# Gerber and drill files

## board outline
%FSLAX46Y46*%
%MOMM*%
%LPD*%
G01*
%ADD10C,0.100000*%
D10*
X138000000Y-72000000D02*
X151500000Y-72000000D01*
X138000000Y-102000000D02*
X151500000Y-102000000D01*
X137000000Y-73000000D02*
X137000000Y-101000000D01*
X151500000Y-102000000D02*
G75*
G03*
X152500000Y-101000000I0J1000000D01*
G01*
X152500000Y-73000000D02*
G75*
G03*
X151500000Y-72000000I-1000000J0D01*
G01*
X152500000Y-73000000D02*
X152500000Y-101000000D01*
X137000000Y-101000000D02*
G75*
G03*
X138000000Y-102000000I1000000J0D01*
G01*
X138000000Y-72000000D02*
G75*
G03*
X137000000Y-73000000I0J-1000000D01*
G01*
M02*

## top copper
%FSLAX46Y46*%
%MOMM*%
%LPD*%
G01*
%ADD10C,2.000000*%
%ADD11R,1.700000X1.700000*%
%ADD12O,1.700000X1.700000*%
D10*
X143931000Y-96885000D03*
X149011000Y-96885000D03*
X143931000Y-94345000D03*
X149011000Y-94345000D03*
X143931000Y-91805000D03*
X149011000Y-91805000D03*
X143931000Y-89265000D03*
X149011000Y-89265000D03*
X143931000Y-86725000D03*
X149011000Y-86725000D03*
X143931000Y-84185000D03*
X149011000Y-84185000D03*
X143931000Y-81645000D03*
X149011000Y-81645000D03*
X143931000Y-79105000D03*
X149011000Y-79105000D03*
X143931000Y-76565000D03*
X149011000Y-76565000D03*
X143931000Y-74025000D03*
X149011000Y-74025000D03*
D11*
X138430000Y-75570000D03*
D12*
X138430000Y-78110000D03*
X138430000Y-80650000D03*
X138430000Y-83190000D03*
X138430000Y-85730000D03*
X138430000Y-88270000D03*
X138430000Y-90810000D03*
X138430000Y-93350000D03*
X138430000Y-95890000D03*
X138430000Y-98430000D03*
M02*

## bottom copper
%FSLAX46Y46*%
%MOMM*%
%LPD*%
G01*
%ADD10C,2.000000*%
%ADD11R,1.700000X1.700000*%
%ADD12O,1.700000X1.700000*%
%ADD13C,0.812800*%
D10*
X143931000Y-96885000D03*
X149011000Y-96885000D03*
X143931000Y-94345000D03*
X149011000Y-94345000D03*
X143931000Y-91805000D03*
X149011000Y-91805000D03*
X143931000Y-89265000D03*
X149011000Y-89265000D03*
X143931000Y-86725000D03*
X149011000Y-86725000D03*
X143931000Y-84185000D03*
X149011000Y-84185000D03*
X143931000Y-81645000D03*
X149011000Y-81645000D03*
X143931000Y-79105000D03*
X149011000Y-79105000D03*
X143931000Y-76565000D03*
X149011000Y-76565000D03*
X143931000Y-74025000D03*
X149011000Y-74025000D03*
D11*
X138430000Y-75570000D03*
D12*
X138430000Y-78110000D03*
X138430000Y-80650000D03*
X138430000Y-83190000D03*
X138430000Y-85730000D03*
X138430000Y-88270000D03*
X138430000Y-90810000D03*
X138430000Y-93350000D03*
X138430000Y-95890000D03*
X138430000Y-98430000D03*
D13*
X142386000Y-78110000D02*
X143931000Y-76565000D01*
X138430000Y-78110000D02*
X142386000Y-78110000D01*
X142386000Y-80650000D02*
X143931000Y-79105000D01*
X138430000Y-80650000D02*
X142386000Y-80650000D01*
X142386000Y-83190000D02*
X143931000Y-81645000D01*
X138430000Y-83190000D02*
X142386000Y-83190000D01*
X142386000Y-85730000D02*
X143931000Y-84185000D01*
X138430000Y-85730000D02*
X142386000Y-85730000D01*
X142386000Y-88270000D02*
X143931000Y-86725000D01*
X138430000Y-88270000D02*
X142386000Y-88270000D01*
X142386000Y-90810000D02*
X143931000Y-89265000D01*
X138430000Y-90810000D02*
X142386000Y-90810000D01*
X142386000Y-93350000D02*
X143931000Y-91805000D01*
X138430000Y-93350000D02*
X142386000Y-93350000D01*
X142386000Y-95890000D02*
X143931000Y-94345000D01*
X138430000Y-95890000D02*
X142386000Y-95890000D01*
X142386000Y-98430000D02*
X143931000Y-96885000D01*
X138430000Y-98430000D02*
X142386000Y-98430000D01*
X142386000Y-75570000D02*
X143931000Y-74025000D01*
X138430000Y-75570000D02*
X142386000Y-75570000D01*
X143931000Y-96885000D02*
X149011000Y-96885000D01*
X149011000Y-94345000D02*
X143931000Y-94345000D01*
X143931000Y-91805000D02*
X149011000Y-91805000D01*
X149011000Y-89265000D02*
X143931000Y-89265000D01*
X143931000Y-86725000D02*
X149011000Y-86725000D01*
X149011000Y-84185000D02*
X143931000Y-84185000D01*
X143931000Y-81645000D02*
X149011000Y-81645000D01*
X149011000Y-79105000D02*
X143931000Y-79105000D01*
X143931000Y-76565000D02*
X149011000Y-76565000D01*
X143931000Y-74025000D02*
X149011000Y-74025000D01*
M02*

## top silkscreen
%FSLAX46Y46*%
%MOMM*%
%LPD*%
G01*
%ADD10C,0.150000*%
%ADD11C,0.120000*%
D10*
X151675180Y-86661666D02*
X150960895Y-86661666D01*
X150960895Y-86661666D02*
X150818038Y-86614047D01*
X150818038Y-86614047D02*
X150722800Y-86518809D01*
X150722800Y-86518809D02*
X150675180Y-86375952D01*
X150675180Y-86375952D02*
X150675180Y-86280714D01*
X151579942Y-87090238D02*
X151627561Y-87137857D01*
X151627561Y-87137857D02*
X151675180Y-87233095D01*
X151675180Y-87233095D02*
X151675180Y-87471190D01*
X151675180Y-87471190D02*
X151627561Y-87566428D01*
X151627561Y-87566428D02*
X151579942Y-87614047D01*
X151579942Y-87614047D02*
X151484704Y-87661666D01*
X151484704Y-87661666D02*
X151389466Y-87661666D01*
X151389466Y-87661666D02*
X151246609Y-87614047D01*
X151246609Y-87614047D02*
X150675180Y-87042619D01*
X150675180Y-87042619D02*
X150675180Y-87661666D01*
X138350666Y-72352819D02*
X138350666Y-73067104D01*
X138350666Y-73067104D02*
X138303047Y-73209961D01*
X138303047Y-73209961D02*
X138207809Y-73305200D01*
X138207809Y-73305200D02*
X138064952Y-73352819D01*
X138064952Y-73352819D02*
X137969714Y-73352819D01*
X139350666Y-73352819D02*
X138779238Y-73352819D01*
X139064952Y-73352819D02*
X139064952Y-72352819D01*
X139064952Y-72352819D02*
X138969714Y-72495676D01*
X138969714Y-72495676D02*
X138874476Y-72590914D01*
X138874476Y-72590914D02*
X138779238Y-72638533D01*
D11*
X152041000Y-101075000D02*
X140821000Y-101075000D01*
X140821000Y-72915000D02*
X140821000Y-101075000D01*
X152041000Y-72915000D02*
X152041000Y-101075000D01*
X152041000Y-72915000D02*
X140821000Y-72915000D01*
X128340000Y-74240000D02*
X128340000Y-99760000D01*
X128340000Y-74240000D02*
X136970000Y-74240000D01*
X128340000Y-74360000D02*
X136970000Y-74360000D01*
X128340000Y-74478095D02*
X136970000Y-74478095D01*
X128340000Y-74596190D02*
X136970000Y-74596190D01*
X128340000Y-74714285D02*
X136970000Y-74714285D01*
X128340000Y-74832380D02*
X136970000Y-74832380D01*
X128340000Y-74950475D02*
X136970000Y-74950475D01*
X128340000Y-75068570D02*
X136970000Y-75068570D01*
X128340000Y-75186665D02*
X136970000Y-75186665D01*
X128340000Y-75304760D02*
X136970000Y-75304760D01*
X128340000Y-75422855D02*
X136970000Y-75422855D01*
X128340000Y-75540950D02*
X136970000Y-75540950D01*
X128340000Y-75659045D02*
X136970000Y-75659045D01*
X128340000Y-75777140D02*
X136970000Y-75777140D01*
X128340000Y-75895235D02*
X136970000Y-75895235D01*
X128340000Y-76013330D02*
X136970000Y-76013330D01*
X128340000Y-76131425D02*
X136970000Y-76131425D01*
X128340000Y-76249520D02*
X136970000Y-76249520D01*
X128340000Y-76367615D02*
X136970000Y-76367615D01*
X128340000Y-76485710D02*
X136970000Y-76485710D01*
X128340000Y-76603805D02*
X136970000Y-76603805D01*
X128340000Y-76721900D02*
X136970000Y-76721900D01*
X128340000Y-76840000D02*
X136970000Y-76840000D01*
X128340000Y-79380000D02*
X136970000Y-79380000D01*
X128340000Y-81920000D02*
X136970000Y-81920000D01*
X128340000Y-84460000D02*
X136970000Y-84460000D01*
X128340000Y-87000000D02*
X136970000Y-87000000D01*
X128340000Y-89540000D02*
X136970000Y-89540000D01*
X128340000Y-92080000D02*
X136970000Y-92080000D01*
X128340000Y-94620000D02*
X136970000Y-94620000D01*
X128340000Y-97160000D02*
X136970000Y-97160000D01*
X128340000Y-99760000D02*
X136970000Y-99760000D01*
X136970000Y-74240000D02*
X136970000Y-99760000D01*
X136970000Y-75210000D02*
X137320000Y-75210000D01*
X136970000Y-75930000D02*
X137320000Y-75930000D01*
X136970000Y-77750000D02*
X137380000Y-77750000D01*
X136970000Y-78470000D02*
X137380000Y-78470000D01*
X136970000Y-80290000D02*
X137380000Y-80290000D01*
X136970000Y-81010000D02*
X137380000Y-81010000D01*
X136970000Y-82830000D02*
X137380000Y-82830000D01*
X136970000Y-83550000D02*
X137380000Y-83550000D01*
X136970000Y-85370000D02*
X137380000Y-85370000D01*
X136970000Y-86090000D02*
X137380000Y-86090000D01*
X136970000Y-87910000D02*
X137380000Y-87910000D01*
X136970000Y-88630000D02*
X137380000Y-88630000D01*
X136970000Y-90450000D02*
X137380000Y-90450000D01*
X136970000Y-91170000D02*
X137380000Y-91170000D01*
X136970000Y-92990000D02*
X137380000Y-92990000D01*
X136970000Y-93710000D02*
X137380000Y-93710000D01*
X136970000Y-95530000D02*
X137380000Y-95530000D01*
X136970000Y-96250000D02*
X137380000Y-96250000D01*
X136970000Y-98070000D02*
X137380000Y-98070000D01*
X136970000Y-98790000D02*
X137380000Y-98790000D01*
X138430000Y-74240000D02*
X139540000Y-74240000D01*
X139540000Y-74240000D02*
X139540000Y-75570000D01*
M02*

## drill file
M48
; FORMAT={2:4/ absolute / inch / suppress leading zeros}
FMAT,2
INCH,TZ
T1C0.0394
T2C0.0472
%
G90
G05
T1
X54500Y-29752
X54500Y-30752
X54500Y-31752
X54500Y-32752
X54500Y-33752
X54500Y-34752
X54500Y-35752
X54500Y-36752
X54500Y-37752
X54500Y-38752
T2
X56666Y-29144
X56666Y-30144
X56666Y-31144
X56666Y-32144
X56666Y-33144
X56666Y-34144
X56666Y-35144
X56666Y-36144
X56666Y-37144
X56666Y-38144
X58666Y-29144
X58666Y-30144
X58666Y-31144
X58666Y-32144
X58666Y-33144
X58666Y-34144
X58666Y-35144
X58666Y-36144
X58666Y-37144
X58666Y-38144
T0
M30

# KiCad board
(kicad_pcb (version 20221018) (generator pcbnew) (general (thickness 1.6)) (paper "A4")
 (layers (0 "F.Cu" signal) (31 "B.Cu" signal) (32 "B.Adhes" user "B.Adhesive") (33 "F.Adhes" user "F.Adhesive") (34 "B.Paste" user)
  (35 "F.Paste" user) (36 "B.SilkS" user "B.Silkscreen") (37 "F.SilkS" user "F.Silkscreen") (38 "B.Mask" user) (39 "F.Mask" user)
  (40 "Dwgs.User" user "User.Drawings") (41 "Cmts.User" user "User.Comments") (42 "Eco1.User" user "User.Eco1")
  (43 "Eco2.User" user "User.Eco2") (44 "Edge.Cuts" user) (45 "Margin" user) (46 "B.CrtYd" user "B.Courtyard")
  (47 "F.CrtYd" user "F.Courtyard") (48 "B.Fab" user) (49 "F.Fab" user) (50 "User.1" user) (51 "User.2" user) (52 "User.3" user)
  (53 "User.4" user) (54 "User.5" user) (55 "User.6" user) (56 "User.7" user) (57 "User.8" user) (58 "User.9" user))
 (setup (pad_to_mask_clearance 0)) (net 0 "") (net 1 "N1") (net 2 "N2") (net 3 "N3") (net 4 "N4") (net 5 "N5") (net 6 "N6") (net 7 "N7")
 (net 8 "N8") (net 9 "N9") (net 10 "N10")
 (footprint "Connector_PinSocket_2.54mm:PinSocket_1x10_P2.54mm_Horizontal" (layer "F.Cu") (at 138.43 75.57)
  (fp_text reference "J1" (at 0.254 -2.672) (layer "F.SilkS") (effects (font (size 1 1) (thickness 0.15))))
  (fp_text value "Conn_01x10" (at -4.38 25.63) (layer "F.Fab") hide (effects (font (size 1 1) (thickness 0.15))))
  (fp_line (start -10.09 -1.33) (end -10.09 24.19) (stroke (width 0.12) (type solid)) (layer "F.SilkS"))
  (fp_line (start -10.09 -1.33) (end -1.46 -1.33) (stroke (width 0.12) (type solid)) (layer "F.SilkS"))
  (fp_line (start -10.09 -1.21) (end -1.46 -1.21) (stroke (width 0.12) (type solid)) (layer "F.SilkS"))
  (fp_line (start -10.09 -1.091905) (end -1.46 -1.091905) (stroke (width 0.12) (type solid)) (layer "F.SilkS"))
  (fp_line (start -10.09 -0.97381) (end -1.46 -0.97381) (stroke (width 0.12) (type solid)) (layer "F.SilkS"))
  (fp_line (start -10.09 -0.855715) (end -1.46 -0.855715) (stroke (width 0.12) (type solid)) (layer "F.SilkS"))
  (fp_line (start -10.09 -0.73762) (end -1.46 -0.73762) (stroke (width 0.12) (type solid)) (layer "F.SilkS"))
  (fp_line (start -10.09 -0.619525) (end -1.46 -0.619525) (stroke (width 0.12) (type solid)) (layer "F.SilkS"))
  (fp_line (start -10.09 -0.50143) (end -1.46 -0.50143) (stroke (width 0.12) (type solid)) (layer "F.SilkS"))
  (fp_line (start -10.09 -0.383335) (end -1.46 -0.383335) (stroke (width 0.12) (type solid)) (layer "F.SilkS"))
  (fp_line (start -10.09 -0.26524) (end -1.46 -0.26524) (stroke (width 0.12) (type solid)) (layer "F.SilkS"))
  (fp_line (start -10.09 -0.147145) (end -1.46 -0.147145) (stroke (width 0.12) (type solid)) (layer "F.SilkS"))
  (fp_line (start -10.09 -0.02905) (end -1.46 -0.02905) (stroke (width 0.12) (type solid)) (layer "F.SilkS"))
  (fp_line (start -10.09 0.089045) (end -1.46 0.089045) (stroke (width 0.12) (type solid)) (layer "F.SilkS"))
  (fp_line (start -10.09 0.20714) (end -1.46 0.20714) (stroke (width 0.12) (type solid)) (layer "F.SilkS"))
  (fp_line (start -10.09 0.325235) (end -1.46 0.325235) (stroke (width 0.12) (type solid)) (layer "F.SilkS"))
  (fp_line (start -10.09 0.44333) (end -1.46 0.44333) (stroke (width 0.12) (type solid)) (layer "F.SilkS"))
  (fp_line (start -10.09 0.561425) (end -1.46 0.561425) (stroke (width 0.12) (type solid)) (layer "F.SilkS"))
  (fp_line (start -10.09 0.67952) (end -1.46 0.67952) (stroke (width 0.12) (type solid)) (layer "F.SilkS"))
  (fp_line (start -10.09 0.797615) (end -1.46 0.797615) (stroke (width 0.12) (type solid)) (layer "F.SilkS"))
  (fp_line (start -10.09 0.91571) (end -1.46 0.91571) (stroke (width 0.12) (type solid)) (layer "F.SilkS"))
  (fp_line (start -10.09 1.033805) (end -1.46 1.033805) (stroke (width 0.12) (type solid)) (layer "F.SilkS"))
  (fp_line (start -10.09 1.1519) (end -1.46 1.1519) (stroke (width 0.12) (type solid)) (layer "F.SilkS"))
  (fp_line (start -10.09 1.27) (end -1.46 1.27) (stroke (width 0.12) (type solid)) (layer "F.SilkS"))
  (fp_line (start -10.09 3.81) (end -1.46 3.81) (stroke (width 0.12) (type solid)) (layer "F.SilkS"))
  (fp_line (start -10.09 6.35) (end -1.46 6.35) (stroke (width 0.12) (type solid)) (layer "F.SilkS"))
  (fp_line (start -10.09 8.89) (end -1.46 8.89) (stroke (width 0.12) (type solid)) (layer "F.SilkS"))
  (fp_line (start -10.09 11.43) (end -1.46 11.43) (stroke (width 0.12) (type solid)) (layer "F.SilkS"))
  (fp_line (start -10.09 13.97) (end -1.46 13.97) (stroke (width 0.12) (type solid)) (layer "F.SilkS"))
  (fp_line (start -10.09 16.51) (end -1.46 16.51) (stroke (width 0.12) (type solid)) (layer "F.SilkS"))
  (fp_line (start -10.09 19.05) (end -1.46 19.05) (stroke (width 0.12) (type solid)) (layer "F.SilkS"))
  (fp_line (start -10.09 21.59) (end -1.46 21.59) (stroke (width 0.12) (type solid)) (layer "F.SilkS"))
  (fp_line (start -10.09 24.19) (end -1.46 24.19) (stroke (width 0.12) (type solid)) (layer "F.SilkS"))
  (fp_line (start -1.46 -1.33) (end -1.46 24.19) (stroke (width 0.12) (type solid)) (layer "F.SilkS"))
  (fp_line (start -1.46 -0.36) (end -1.11 -0.36) (stroke (width 0.12) (type solid)) (layer "F.SilkS"))
  (fp_line (start -1.46 0.36) (end -1.11 0.36) (stroke (width 0.12) (type solid)) (layer "F.SilkS"))
  (fp_line (start -1.46 2.18) (end -1.05 2.18) (stroke (width 0.12) (type solid)) (layer "F.SilkS"))
  (fp_line (start -1.46 2.9) (end -1.05 2.9) (stroke (width 0.12) (type solid)) (layer "F.SilkS"))
  (fp_line (start -1.46 4.72) (end -1.05 4.72) (stroke (width 0.12) (type solid)) (layer "F.SilkS"))
  (fp_line (start -1.46 5.44) (end -1.05 5.44) (stroke (width 0.12) (type solid)) (layer "F.SilkS"))
  (fp_line (start -1.46 7.26) (end -1.05 7.26) (stroke (width 0.12) (type solid)) (layer "F.SilkS"))
  (fp_line (start -1.46 7.98) (end -1.05 7.98) (stroke (width 0.12) (type solid)) (layer "F.SilkS"))
  (fp_line (start -1.46 9.8) (end -1.05 9.8) (stroke (width 0.12) (type solid)) (layer "F.SilkS"))
  (fp_line (start -1.46 10.52) (end -1.05 10.52) (stroke (width 0.12) (type solid)) (layer "F.SilkS"))
  (fp_line (start -1.46 12.34) (end -1.05 12.34) (stroke (width 0.12) (type solid)) (layer "F.SilkS"))
  (fp_line (start -1.46 13.06) (end -1.05 13.06) (stroke (width 0.12) (type solid)) (layer "F.SilkS"))
  (fp_line (start -1.46 14.88) (end -1.05 14.88) (stroke (width 0.12) (type solid)) (layer "F.SilkS"))
  (fp_line (start -1.46 15.6) (end -1.05 15.6) (stroke (width 0.12) (type solid)) (layer "F.SilkS"))
  (fp_line (start -1.46 17.42) (end -1.05 17.42) (stroke (width 0.12) (type solid)) (layer "F.SilkS"))
  (fp_line (start -1.46 18.14) (end -1.05 18.14) (stroke (width 0.12) (type solid)) (layer "F.SilkS"))
  (fp_line (start -1.46 19.96) (end -1.05 19.96) (stroke (width 0.12) (type solid)) (layer "F.SilkS"))
  (fp_line (start -1.46 20.68) (end -1.05 20.68) (stroke (width 0.12) (type solid)) (layer "F.SilkS"))
  (fp_line (start -1.46 22.5) (end -1.05 22.5) (stroke (width 0.12) (type solid)) (layer "F.SilkS"))
  (fp_line (start -1.46 23.22) (end -1.05 23.22) (stroke (width 0.12) (type solid)) (layer "F.SilkS"))
  (fp_line (start 0 -1.33) (end 1.11 -1.33) (stroke (width 0.12) (type solid)) (layer "F.SilkS"))
  (fp_line (start 1.11 -1.33) (end 1.11 0) (stroke (width 0.12) (type solid)) (layer "F.SilkS"))
  (pad "1" thru_hole rect (at 0 0) (size 1.7 1.7) (drill 1) (layers "*.Cu" "*.Mask") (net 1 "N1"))
  (pad "2" thru_hole oval (at 0 2.54) (size 1.7 1.7) (drill 1) (layers "*.Cu" "*.Mask") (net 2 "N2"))
  (pad "3" thru_hole oval (at 0 5.08) (size 1.7 1.7) (drill 1) (layers "*.Cu" "*.Mask") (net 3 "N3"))
  (pad "4" thru_hole oval (at 0 7.62) (size 1.7 1.7) (drill 1) (layers "*.Cu" "*.Mask") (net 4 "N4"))
  (pad "5" thru_hole oval (at 0 10.16) (size 1.7 1.7) (drill 1) (layers "*.Cu" "*.Mask") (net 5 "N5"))
  (pad "6" thru_hole oval (at 0 12.7) (size 1.7 1.7) (drill 1) (layers "*.Cu" "*.Mask") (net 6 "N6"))
  (pad "7" thru_hole oval (at 0 15.24) (size 1.7 1.7) (drill 1) (layers "*.Cu" "*.Mask") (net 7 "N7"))
  (pad "8" thru_hole oval (at 0 17.78) (size 1.7 1.7) (drill 1) (layers "*.Cu" "*.Mask") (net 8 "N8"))
  (pad "9" thru_hole oval (at 0 20.32) (size 1.7 1.7) (drill 1) (layers "*.Cu" "*.Mask") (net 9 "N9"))
  (pad "10" thru_hole oval (at 0 22.86) (size 1.7 1.7) (drill 1) (layers "*.Cu" "*.Mask") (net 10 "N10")))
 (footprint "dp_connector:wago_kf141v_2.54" (layer "F.Cu") (at 146.431 86.995 -90)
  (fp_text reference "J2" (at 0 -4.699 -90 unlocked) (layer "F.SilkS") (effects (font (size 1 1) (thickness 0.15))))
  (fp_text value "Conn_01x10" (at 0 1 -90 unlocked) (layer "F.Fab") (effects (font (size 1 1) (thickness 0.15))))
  (fp_line (start -14.08 -5.61) (end -14.08 5.61) (stroke (width 0.12) (type default)) (layer "F.SilkS"))
  (fp_line (start -14.08 -5.61) (end 14.08 -5.61) (stroke (width 0.12) (type default)) (layer "F.SilkS"))
  (fp_line (start -14.08 5.61) (end 14.08 5.61) (stroke (width 0.12) (type default)) (layer "F.SilkS"))
  (fp_line (start 14.08 -5.61) (end 14.08 5.61) (stroke (width 0.12) (type default)) (layer "F.SilkS"))
  (pad "1" thru_hole circle (at -12.97 -2.58 270) (size 2 2) (drill 1.2) (layers "*.Cu" "*.Mask") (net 1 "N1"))
  (pad "1" thru_hole circle (at -12.97 2.5 270) (size 2 2) (drill 1.2) (layers "*.Cu" "*.Mask") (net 1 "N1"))
  (pad "2" thru_hole circle (at -10.43 -2.58 270) (size 2 2) (drill 1.2) (layers "*.Cu" "*.Mask") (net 2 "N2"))
  (pad "2" thru_hole circle (at -10.43 2.5 270) (size 2 2) (drill 1.2) (layers "*.Cu" "*.Mask") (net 2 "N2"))
  (pad "3" thru_hole circle (at -7.89 -2.58 270) (size 2 2) (drill 1.2) (layers "*.Cu" "*.Mask") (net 3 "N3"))
  (pad "3" thru_hole circle (at -7.89 2.5 270) (size 2 2) (drill 1.2) (layers "*.Cu" "*.Mask") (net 3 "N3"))
  (pad "4" thru_hole circle (at -5.35 -2.58 270) (size 2 2) (drill 1.2) (layers "*.Cu" "*.Mask") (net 4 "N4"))
  (pad "4" thru_hole circle (at -5.35 2.5 270) (size 2 2) (drill 1.2) (layers "*.Cu" "*.Mask") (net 4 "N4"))
  (pad "5" thru_hole circle (at -2.81 -2.58 270) (size 2 2) (drill 1.2) (layers "*.Cu" "*.Mask") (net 5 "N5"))
  (pad "5" thru_hole circle (at -2.81 2.5 270) (size 2 2) (drill 1.2) (layers "*.Cu" "*.Mask") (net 5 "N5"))
  (pad "6" thru_hole circle (at -0.27 -2.58 270) (size 2 2) (drill 1.2) (layers "*.Cu" "*.Mask") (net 6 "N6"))
  (pad "6" thru_hole circle (at -0.27 2.5 270) (size 2 2) (drill 1.2) (layers "*.Cu" "*.Mask") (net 6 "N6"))
  (pad "7" thru_hole circle (at 2.27 -2.58 270) (size 2 2) (drill 1.2) (layers "*.Cu" "*.Mask") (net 7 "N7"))
  (pad "7" thru_hole circle (at 2.27 2.5 270) (size 2 2) (drill 1.2) (layers "*.Cu" "*.Mask") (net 7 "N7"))
  (pad "8" thru_hole circle (at 4.81 -2.58 270) (size 2 2) (drill 1.2) (layers "*.Cu" "*.Mask") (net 8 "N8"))
  (pad "8" thru_hole circle (at 4.81 2.5 270) (size 2 2) (drill 1.2) (layers "*.Cu" "*.Mask") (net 8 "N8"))
  (pad "9" thru_hole circle (at 7.35 -2.58 270) (size 2 2) (drill 1.2) (layers "*.Cu" "*.Mask") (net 9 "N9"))
  (pad "9" thru_hole circle (at 7.35 2.5 270) (size 2 2) (drill 1.2) (layers "*.Cu" "*.Mask") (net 9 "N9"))
  (pad "10" thru_hole circle (at 9.89 -2.58 270) (size 2 2) (drill 1.2) (layers "*.Cu" "*.Mask") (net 10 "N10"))
  (pad "10" thru_hole circle (at 9.89 2.5 270) (size 2 2) (drill 1.2) (layers "*.Cu" "*.Mask") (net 10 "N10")))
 (gr_line (start 138 72) (end 151.5 72) (stroke (width 0.1) (type default)) (layer "Edge.Cuts"))
 (gr_line (start 138 102) (end 151.5 102) (stroke (width 0.1) (type default)) (layer "Edge.Cuts"))
 (gr_line (start 137 73) (end 137 101) (stroke (width 0.1) (type default)) (layer "Edge.Cuts"))
 (gr_arc (start 152.5 101) (mid 152.207107 101.707107) (end 151.5 102) (stroke (width 0.1) (type default)) (layer "Edge.Cuts"))
 (gr_arc (start 151.5 72) (mid 152.207107 72.292893) (end 152.5 73) (stroke (width 0.1) (type default)) (layer "Edge.Cuts"))
 (gr_line (start 152.5 73) (end 152.5 101) (stroke (width 0.1) (type default)) (layer "Edge.Cuts"))
 (gr_arc (start 138 102) (mid 137.292893 101.707107) (end 137 101) (stroke (width 0.1) (type default)) (layer "Edge.Cuts"))
 (gr_arc (start 137 73) (mid 137.292893 72.292893) (end 138 72) (stroke (width 0.1) (type default)) (layer "Edge.Cuts"))
 (segment (start 138.43 75.57) (end 142.386 75.57) (width 0.8128) (layer "B.Cu") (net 1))
 (segment (start 142.386 75.57) (end 143.931 74.025) (width 0.8128) (layer "B.Cu") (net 1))
 (segment (start 143.931 74.025) (end 149.011 74.025) (width 0.8128) (layer "B.Cu") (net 1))
 (segment (start 138.43 78.11) (end 142.386 78.11) (width 0.8128) (layer "B.Cu") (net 2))
 (segment (start 143.931 76.565) (end 149.011 76.565) (width 0.8128) (layer "B.Cu") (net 2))
 (segment (start 142.386 78.11) (end 143.931 76.565) (width 0.8128) (layer "B.Cu") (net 2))
 (segment (start 149.011 79.105) (end 143.931 79.105) (width 0.8128) (layer "B.Cu") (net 3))
 (segment (start 142.386 80.65) (end 143.931 79.105) (width 0.8128) (layer "B.Cu") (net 3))
 (segment (start 138.43 80.65) (end 142.386 80.65) (width 0.8128) (layer "B.Cu") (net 3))
 (segment (start 138.43 83.19) (end 142.386 83.19) (width 0.8128) (layer "B.Cu") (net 4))
 (segment (start 143.931 81.645) (end 149.011 81.645) (width 0.8128) (layer "B.Cu") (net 4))
 (segment (start 142.386 83.19) (end 143.931 81.645) (width 0.8128) (layer "B.Cu") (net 4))
 (segment (start 142.386 85.73) (end 143.931 84.185) (width 0.8128) (layer "B.Cu") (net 5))
 (segment (start 149.011 84.185) (end 143.931 84.185) (width 0.8128) (layer "B.Cu") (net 5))
 (segment (start 138.43 85.73) (end 142.386 85.73) (width 0.8128) (layer "B.Cu") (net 5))
 (segment (start 143.931 86.725) (end 149.011 86.725) (width 0.8128) (layer "B.Cu") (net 6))
 (segment (start 142.386 88.27) (end 143.931 86.725) (width 0.8128) (layer "B.Cu") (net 6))
 (segment (start 138.43 88.27) (end 142.386 88.27) (width 0.8128) (layer "B.Cu") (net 6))
 (segment (start 142.386 90.81) (end 143.931 89.265) (width 0.8128) (layer "B.Cu") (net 7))
 (segment (start 138.43 90.81) (end 142.386 90.81) (width 0.8128) (layer "B.Cu") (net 7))
 (segment (start 149.011 89.265) (end 143.931 89.265) (width 0.8128) (layer "B.Cu") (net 7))
 (segment (start 142.386 93.35) (end 143.931 91.805) (width 0.8128) (layer "B.Cu") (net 8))
 (segment (start 138.43 93.35) (end 142.386 93.35) (width 0.8128) (layer "B.Cu") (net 8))
 (segment (start 143.931 91.805) (end 149.011 91.805) (width 0.8128) (layer "B.Cu") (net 8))
 (segment (start 142.386 95.89) (end 143.931 94.345) (width 0.8128) (layer "B.Cu") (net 9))
 (segment (start 138.43 95.89) (end 142.386 95.89) (width 0.8128) (layer "B.Cu") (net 9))
 (segment (start 149.011 94.345) (end 143.931 94.345) (width 0.8128) (layer "B.Cu") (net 9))
 (segment (start 138.43 98.43) (end 142.386 98.43) (width 0.8128) (layer "B.Cu") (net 10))
 (segment (start 142.386 98.43) (end 143.931 96.885) (width 0.8128) (layer "B.Cu") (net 10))
 (segment (start 143.931 96.885) (end 149.011 96.885) (width 0.8128) (layer "B.Cu") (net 10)))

